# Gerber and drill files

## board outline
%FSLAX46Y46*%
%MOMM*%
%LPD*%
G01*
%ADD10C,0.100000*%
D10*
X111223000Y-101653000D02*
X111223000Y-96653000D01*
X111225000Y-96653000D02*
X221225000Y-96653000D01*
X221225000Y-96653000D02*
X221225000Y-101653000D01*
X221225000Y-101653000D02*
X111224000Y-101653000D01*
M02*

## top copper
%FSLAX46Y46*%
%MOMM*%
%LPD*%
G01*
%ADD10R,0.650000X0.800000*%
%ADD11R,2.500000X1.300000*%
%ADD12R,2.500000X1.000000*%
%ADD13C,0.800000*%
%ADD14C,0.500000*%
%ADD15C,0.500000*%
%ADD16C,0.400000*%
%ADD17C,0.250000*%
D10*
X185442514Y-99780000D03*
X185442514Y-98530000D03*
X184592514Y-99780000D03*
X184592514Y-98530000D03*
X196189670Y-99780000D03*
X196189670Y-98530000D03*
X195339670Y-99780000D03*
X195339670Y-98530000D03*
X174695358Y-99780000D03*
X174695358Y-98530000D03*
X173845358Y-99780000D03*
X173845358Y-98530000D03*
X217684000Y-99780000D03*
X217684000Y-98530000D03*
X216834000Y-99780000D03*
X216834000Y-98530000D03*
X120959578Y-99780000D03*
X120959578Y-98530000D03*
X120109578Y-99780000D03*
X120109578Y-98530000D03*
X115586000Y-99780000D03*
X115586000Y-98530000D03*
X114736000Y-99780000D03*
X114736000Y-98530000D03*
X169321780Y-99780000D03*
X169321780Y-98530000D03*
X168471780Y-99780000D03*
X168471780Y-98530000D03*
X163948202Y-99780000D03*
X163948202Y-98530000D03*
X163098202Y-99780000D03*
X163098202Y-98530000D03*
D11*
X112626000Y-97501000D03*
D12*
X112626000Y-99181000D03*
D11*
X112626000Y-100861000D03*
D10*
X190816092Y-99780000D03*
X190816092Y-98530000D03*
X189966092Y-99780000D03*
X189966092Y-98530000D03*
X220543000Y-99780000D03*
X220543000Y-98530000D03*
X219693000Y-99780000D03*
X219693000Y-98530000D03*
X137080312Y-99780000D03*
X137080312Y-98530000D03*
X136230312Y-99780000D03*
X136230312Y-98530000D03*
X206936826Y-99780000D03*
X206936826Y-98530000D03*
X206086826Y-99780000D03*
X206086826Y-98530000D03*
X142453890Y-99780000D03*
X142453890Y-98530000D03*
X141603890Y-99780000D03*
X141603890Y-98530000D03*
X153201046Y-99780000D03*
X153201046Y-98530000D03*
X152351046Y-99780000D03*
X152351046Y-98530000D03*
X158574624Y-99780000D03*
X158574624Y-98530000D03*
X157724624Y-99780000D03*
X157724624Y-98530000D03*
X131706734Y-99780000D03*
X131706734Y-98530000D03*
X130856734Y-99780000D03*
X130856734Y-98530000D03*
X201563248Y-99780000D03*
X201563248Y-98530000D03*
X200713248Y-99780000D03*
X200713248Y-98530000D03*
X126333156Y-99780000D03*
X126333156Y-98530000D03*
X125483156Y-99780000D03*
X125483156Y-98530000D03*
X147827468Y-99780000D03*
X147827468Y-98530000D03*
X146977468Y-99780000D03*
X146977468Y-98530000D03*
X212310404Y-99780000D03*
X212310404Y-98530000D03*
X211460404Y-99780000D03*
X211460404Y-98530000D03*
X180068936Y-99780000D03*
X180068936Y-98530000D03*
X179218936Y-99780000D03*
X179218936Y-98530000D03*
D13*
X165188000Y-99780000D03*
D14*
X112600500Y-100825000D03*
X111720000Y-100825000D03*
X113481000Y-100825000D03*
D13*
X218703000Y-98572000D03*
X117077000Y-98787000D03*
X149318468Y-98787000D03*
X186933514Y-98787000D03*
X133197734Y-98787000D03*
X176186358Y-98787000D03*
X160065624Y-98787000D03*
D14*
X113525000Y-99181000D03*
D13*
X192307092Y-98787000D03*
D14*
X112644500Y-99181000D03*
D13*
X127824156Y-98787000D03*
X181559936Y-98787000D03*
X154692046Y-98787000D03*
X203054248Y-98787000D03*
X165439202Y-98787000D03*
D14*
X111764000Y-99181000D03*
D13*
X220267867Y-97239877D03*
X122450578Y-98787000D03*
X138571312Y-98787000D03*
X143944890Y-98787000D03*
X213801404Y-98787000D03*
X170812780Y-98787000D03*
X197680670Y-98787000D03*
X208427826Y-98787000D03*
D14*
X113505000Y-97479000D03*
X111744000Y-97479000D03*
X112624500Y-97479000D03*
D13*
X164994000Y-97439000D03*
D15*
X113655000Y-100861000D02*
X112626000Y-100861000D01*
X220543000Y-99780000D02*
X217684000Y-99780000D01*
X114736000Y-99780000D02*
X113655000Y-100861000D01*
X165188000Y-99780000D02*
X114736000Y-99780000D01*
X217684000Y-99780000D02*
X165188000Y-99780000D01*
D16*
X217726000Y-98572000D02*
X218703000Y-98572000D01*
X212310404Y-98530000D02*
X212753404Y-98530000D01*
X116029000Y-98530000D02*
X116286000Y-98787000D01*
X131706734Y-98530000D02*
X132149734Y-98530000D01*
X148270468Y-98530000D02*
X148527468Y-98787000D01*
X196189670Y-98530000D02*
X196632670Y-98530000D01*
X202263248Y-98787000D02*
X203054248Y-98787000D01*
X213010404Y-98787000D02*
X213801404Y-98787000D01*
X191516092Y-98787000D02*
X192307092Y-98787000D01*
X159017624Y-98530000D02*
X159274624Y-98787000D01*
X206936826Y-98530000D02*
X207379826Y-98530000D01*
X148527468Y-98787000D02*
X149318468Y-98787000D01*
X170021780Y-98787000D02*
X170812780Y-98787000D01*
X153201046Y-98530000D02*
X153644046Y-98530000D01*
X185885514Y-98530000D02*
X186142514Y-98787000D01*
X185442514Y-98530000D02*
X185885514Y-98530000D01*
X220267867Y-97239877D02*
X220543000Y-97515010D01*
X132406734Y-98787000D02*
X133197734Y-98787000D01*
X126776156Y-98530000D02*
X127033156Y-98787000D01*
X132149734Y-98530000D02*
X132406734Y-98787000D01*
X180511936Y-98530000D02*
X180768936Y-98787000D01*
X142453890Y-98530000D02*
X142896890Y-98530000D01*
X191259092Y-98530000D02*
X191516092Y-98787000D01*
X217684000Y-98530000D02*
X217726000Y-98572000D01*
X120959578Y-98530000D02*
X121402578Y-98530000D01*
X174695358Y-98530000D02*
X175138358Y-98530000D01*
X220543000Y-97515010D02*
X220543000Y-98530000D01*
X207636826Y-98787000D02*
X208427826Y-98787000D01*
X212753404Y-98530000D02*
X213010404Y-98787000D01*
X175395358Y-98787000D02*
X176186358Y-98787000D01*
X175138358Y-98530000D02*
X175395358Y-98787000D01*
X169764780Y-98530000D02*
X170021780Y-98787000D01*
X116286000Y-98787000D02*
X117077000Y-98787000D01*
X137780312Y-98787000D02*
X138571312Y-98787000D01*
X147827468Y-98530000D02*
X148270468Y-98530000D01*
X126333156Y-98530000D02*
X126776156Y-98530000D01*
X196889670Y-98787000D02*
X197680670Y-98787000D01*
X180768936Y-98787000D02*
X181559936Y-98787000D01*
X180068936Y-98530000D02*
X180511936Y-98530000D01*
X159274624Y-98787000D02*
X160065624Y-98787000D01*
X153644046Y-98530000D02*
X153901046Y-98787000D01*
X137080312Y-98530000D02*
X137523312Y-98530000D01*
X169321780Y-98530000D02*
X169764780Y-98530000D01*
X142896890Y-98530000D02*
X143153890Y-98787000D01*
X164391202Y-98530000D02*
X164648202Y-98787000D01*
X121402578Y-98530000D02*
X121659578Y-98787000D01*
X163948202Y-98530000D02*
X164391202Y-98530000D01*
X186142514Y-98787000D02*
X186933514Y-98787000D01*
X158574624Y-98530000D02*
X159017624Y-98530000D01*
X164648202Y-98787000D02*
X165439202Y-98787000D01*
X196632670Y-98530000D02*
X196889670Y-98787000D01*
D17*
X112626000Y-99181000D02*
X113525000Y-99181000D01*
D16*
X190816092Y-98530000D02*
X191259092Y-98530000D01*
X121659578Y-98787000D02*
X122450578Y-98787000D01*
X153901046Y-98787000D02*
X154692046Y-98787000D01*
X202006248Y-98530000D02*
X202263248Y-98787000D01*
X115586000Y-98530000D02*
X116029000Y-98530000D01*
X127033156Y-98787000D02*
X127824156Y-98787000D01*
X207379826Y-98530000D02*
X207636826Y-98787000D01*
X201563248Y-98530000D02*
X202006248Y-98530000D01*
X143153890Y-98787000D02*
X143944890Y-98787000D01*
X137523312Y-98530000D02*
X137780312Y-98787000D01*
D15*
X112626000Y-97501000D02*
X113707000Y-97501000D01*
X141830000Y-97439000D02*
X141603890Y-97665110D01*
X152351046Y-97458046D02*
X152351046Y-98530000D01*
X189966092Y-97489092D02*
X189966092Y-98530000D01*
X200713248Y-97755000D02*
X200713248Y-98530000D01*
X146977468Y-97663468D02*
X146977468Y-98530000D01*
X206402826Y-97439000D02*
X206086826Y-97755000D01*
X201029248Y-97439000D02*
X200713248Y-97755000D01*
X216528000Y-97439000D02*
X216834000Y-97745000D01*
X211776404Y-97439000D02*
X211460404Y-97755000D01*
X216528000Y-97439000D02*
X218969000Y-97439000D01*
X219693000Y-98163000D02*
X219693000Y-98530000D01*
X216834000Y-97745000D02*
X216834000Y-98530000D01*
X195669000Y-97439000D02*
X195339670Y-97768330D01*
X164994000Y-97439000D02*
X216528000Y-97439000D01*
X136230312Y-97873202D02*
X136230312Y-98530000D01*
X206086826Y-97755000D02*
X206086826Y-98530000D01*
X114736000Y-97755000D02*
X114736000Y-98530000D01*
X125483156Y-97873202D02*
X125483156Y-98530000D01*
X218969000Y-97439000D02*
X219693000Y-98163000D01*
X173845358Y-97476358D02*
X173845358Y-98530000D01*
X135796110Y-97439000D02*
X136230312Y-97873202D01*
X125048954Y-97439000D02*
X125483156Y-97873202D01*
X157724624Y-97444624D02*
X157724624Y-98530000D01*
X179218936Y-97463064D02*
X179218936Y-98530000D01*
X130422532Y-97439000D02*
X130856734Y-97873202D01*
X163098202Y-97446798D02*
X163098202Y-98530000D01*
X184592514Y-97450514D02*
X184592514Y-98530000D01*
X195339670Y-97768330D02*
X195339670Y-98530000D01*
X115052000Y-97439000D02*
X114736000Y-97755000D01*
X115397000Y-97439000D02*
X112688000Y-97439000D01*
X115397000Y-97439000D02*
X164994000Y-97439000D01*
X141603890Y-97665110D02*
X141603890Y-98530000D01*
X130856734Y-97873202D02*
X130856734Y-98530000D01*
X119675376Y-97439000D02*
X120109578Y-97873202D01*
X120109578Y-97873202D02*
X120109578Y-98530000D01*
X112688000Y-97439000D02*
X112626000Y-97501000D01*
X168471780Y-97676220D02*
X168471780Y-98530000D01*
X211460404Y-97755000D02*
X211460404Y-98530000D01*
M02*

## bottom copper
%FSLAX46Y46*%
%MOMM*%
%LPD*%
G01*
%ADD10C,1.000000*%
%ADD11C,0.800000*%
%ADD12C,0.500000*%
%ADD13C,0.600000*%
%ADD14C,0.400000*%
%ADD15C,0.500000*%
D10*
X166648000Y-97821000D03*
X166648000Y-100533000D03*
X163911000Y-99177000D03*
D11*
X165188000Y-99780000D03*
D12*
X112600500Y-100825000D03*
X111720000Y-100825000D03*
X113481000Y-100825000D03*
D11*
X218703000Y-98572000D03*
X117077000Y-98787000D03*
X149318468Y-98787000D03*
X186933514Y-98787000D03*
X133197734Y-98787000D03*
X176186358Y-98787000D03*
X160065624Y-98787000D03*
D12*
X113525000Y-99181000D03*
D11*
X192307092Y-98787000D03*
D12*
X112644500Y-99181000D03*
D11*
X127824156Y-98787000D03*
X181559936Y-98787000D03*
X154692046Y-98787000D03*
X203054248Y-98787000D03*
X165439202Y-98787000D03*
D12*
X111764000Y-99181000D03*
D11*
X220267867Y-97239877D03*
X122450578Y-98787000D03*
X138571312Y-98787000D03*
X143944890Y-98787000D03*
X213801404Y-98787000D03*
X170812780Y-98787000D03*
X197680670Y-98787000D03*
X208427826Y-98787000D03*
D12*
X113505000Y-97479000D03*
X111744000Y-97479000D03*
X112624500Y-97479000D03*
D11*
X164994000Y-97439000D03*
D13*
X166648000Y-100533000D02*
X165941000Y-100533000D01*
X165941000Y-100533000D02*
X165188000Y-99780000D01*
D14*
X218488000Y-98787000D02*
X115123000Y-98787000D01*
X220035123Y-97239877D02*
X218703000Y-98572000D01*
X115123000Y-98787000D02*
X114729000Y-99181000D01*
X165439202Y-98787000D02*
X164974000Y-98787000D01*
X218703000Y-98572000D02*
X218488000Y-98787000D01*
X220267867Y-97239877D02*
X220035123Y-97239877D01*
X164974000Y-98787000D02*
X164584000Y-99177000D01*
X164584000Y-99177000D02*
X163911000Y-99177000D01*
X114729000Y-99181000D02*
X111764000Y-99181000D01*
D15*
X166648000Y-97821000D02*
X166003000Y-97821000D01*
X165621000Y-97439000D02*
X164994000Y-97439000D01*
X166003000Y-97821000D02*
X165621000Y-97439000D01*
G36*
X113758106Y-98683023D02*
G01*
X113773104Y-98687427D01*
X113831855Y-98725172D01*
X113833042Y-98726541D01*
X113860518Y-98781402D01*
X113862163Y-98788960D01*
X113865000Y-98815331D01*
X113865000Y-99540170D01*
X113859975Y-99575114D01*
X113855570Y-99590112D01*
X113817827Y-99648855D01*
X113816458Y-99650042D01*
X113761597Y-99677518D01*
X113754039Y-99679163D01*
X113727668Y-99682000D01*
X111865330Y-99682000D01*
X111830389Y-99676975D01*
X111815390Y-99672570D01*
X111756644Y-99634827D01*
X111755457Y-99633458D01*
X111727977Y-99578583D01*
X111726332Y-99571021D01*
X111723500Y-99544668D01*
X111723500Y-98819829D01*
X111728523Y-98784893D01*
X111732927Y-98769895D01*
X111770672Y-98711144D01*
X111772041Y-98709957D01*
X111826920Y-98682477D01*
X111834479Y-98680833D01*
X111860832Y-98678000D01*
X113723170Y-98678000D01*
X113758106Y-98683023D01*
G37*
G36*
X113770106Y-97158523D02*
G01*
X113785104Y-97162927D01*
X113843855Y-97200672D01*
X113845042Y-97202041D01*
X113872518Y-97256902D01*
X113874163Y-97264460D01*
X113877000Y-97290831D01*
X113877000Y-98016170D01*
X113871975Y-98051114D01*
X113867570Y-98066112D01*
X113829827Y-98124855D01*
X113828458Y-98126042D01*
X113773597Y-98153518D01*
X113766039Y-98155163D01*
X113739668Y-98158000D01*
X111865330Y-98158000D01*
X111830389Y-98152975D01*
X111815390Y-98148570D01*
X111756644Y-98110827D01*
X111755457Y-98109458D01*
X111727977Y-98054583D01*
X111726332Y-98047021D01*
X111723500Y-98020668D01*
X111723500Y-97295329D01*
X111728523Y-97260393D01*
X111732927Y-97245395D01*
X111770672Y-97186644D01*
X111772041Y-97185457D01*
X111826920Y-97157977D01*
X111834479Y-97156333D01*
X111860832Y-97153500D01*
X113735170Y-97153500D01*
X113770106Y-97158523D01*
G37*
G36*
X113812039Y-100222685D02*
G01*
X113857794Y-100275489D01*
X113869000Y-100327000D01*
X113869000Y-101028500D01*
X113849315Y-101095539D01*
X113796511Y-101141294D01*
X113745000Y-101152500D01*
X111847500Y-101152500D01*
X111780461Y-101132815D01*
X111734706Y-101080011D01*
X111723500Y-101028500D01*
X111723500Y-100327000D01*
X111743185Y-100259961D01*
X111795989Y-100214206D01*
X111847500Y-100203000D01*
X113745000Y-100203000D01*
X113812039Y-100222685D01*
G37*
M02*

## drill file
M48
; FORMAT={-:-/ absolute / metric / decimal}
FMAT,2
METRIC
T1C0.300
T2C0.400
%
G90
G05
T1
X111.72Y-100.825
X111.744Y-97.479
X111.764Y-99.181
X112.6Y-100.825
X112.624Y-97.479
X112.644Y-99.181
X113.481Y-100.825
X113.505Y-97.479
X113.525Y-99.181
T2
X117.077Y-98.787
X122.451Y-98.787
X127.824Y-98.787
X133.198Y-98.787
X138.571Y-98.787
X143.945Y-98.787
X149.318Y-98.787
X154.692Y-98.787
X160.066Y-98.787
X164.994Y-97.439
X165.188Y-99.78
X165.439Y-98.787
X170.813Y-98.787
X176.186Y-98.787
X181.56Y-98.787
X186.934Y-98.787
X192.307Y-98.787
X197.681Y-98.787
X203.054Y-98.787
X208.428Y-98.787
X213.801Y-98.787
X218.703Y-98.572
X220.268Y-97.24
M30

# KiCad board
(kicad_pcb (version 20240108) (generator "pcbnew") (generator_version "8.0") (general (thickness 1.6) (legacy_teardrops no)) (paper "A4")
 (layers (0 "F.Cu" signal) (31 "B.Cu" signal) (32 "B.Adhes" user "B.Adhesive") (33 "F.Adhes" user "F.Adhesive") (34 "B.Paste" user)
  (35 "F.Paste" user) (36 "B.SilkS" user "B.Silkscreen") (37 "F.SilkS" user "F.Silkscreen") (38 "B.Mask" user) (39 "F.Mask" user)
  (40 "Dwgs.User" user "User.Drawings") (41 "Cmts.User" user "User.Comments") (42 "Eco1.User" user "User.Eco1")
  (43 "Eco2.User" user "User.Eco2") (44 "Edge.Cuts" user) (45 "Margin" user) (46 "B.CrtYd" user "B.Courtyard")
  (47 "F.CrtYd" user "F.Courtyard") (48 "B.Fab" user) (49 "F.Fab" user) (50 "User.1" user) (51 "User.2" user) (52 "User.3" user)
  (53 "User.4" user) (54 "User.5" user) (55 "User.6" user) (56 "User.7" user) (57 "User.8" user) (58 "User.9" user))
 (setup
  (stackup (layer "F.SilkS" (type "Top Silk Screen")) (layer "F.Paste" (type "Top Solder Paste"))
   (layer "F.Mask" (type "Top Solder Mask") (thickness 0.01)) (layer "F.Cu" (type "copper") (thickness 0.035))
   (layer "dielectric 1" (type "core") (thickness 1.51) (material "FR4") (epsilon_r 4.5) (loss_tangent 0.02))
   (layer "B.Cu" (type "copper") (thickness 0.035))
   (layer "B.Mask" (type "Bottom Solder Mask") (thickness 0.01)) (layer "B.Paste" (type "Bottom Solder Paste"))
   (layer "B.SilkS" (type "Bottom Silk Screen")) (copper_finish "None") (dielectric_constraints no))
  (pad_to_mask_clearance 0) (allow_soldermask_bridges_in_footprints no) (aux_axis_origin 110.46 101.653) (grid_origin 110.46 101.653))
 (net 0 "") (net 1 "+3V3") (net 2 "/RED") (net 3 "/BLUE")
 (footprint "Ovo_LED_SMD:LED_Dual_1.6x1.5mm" (layer "F.Cu") (at 185.017514 99.155 90)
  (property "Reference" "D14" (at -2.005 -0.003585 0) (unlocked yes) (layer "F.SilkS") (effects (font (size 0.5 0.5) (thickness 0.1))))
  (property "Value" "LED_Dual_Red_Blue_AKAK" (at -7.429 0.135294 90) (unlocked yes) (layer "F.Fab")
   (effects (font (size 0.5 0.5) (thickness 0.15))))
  (pad "1" smd rect (at -0.625 0.425 90) (size 0.8 0.65) (layers "F.Cu" "F.Paste" "F.Mask") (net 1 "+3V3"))
  (pad "2" smd rect (at 0.625 0.425 90) (size 0.8 0.65) (layers "F.Cu" "F.Paste" "F.Mask") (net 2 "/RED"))
  (pad "3" smd rect (at -0.625 -0.425 90) (size 0.8 0.65) (layers "F.Cu" "F.Paste" "F.Mask") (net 1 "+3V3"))
  (pad "4" smd rect (at 0.625 -0.425 90) (size 0.8 0.65) (layers "F.Cu" "F.Paste" "F.Mask") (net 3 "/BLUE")))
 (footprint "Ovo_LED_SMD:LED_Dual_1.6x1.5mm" (layer "F.Cu") (at 195.76467 99.155 90)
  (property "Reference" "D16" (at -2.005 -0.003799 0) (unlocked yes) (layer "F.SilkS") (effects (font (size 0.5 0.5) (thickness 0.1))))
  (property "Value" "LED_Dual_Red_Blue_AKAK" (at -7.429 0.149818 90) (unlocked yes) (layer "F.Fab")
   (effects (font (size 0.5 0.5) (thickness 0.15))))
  (pad "1" smd rect (at -0.625 0.425 90) (size 0.8 0.65) (layers "F.Cu" "F.Paste" "F.Mask") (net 1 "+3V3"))
  (pad "2" smd rect (at 0.625 0.425 90) (size 0.8 0.65) (layers "F.Cu" "F.Paste" "F.Mask") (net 2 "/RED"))
  (pad "3" smd rect (at -0.625 -0.425 90) (size 0.8 0.65) (layers "F.Cu" "F.Paste" "F.Mask") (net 1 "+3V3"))
  (pad "4" smd rect (at 0.625 -0.425 90) (size 0.8 0.65) (layers "F.Cu" "F.Paste" "F.Mask") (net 3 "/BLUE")))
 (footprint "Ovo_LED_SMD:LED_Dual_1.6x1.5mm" (layer "F.Cu") (at 174.270358 99.155 90)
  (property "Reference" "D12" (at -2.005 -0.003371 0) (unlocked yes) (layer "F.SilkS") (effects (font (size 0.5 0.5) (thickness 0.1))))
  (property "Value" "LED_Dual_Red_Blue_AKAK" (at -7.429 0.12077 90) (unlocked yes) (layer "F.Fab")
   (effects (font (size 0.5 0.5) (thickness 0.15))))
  (pad "1" smd rect (at -0.625 0.425 90) (size 0.8 0.65) (layers "F.Cu" "F.Paste" "F.Mask") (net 1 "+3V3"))
  (pad "2" smd rect (at 0.625 0.425 90) (size 0.8 0.65) (layers "F.Cu" "F.Paste" "F.Mask") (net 2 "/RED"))
  (pad "3" smd rect (at -0.625 -0.425 90) (size 0.8 0.65) (layers "F.Cu" "F.Paste" "F.Mask") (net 1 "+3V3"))
  (pad "4" smd rect (at 0.625 -0.425 90) (size 0.8 0.65) (layers "F.Cu" "F.Paste" "F.Mask") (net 3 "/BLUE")))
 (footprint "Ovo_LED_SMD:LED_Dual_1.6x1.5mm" (layer "F.Cu") (at 217.259 99.155 90)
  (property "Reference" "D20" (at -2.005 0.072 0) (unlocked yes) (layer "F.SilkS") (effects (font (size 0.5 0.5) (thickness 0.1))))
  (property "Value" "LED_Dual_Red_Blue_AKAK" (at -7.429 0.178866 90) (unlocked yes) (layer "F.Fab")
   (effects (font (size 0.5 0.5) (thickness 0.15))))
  (pad "1" smd rect (at -0.625 0.425 90) (size 0.8 0.65) (layers "F.Cu" "F.Paste" "F.Mask") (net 1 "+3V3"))
  (pad "2" smd rect (at 0.625 0.425 90) (size 0.8 0.65) (layers "F.Cu" "F.Paste" "F.Mask") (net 2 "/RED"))
  (pad "3" smd rect (at -0.625 -0.425 90) (size 0.8 0.65) (layers "F.Cu" "F.Paste" "F.Mask") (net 1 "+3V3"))
  (pad "4" smd rect (at 0.625 -0.425 90) (size 0.8 0.65) (layers "F.Cu" "F.Paste" "F.Mask") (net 3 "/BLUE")))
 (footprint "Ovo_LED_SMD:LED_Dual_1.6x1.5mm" (layer "F.Cu") (at 120.534578 99.155 90)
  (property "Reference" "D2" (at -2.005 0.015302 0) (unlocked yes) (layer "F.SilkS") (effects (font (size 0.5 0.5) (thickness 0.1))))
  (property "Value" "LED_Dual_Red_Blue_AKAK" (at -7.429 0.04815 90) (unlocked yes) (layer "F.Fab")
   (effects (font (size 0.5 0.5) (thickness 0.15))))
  (pad "1" smd rect (at -0.625 0.425 90) (size 0.8 0.65) (layers "F.Cu" "F.Paste" "F.Mask") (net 1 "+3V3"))
  (pad "2" smd rect (at 0.625 0.425 90) (size 0.8 0.65) (layers "F.Cu" "F.Paste" "F.Mask") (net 2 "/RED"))
  (pad "3" smd rect (at -0.625 -0.425 90) (size 0.8 0.65) (layers "F.Cu" "F.Paste" "F.Mask") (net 1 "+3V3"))
  (pad "4" smd rect (at 0.625 -0.425 90) (size 0.8 0.65) (layers "F.Cu" "F.Paste" "F.Mask") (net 3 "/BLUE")))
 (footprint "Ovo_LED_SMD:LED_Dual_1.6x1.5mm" (layer "F.Cu") (at 115.161 99.155 90)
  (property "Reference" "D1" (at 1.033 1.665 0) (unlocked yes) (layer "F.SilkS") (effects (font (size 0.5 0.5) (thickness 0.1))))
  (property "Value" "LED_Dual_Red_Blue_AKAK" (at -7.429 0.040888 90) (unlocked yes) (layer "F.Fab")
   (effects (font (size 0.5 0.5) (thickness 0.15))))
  (pad "1" smd rect (at -0.625 0.425 90) (size 0.8 0.65) (layers "F.Cu" "F.Paste" "F.Mask") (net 1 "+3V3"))
  (pad "2" smd rect (at 0.625 0.425 90) (size 0.8 0.65) (layers "F.Cu" "F.Paste" "F.Mask") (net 2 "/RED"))
  (pad "3" smd rect (at -0.625 -0.425 90) (size 0.8 0.65) (layers "F.Cu" "F.Paste" "F.Mask") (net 1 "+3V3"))
  (pad "4" smd rect (at 0.625 -0.425 90) (size 0.8 0.65) (layers "F.Cu" "F.Paste" "F.Mask") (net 3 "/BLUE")))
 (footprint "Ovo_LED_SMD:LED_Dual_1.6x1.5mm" (layer "F.Cu") (at 168.89678 99.155 90)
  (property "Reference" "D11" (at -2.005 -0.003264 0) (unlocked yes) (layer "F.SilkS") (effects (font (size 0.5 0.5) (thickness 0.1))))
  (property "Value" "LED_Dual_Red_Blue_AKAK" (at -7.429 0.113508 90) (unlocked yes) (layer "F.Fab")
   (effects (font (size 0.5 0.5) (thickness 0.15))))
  (pad "1" smd rect (at -0.625 0.425 90) (size 0.8 0.65) (layers "F.Cu" "F.Paste" "F.Mask") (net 1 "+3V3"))
  (pad "2" smd rect (at 0.625 0.425 90) (size 0.8 0.65) (layers "F.Cu" "F.Paste" "F.Mask") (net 2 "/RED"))
  (pad "3" smd rect (at -0.625 -0.425 90) (size 0.8 0.65) (layers "F.Cu" "F.Paste" "F.Mask") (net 1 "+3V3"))
  (pad "4" smd rect (at 0.625 -0.425 90) (size 0.8 0.65) (layers "F.Cu" "F.Paste" "F.Mask") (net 3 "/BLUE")))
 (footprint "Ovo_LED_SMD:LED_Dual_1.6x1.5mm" (layer "F.Cu") (at 163.523202 99.155 90)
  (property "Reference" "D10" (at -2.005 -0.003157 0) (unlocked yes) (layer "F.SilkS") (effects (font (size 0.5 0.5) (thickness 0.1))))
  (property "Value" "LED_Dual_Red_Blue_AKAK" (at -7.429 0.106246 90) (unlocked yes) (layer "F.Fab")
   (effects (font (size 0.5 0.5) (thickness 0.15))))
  (pad "1" smd rect (at -0.625 0.425 90) (size 0.8 0.65) (layers "F.Cu" "F.Paste" "F.Mask") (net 1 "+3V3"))
  (pad "2" smd rect (at 0.625 0.425 90) (size 0.8 0.65) (layers "F.Cu" "F.Paste" "F.Mask") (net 2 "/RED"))
  (pad "3" smd rect (at -0.625 -0.425 90) (size 0.8 0.65) (layers "F.Cu" "F.Paste" "F.Mask") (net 1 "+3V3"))
  (pad "4" smd rect (at 0.625 -0.425 90) (size 0.8 0.65) (layers "F.Cu" "F.Paste" "F.Mask") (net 3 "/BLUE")))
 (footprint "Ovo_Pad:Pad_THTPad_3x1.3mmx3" (layer "F.Cu") (at 112.666 97.511)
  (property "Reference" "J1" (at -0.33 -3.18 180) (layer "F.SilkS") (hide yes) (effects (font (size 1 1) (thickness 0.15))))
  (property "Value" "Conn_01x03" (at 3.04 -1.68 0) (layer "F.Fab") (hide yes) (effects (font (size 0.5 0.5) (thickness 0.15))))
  (pad "1" smd rect (at -0.04 -0.01 180) (size 2.5 1.3) (layers "F.Cu" "F.Paste" "F.Mask") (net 3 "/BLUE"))
  (pad "2" smd rect (at -0.04 1.67 180) (size 2.5 1) (layers "F.Cu" "F.Paste" "F.Mask") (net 2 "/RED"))
  (pad "3" smd rect (at -0.04 3.35 180) (size 2.5 1.3) (layers "F.Cu" "F.Paste" "F.Mask") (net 1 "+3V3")))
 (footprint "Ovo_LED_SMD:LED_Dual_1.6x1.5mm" (layer "F.Cu") (at 190.391092 99.155 90)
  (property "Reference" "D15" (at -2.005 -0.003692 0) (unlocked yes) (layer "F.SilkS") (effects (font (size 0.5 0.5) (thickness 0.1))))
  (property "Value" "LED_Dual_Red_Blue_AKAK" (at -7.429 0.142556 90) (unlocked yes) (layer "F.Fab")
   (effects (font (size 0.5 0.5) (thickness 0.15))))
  (pad "1" smd rect (at -0.625 0.425 90) (size 0.8 0.65) (layers "F.Cu" "F.Paste" "F.Mask") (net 1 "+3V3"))
  (pad "2" smd rect (at 0.625 0.425 90) (size 0.8 0.65) (layers "F.Cu" "F.Paste" "F.Mask") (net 2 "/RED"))
  (pad "3" smd rect (at -0.625 -0.425 90) (size 0.8 0.65) (layers "F.Cu" "F.Paste" "F.Mask") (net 1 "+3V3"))
  (pad "4" smd rect (at 0.625 -0.425 90) (size 0.8 0.65) (layers "F.Cu" "F.Paste" "F.Mask") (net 3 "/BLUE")))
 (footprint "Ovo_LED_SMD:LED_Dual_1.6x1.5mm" (layer "F.Cu") (at 220.118 99.155 90)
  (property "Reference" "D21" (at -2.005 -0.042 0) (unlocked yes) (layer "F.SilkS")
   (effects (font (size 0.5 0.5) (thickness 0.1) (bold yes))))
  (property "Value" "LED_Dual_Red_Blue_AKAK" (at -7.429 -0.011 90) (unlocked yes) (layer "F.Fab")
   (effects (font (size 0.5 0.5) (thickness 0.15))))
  (pad "1" smd rect (at -0.625 0.425 90) (size 0.8 0.65) (layers "F.Cu" "F.Paste" "F.Mask") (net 1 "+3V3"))
  (pad "2" smd rect (at 0.625 0.425 90) (size 0.8 0.65) (layers "F.Cu" "F.Paste" "F.Mask") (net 2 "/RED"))
  (pad "3" smd rect (at -0.625 -0.425 90) (size 0.8 0.65) (layers "F.Cu" "F.Paste" "F.Mask") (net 1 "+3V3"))
  (pad "4" smd rect (at 0.625 -0.425 90) (size 0.8 0.65) (layers "F.Cu" "F.Paste" "F.Mask") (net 3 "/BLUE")))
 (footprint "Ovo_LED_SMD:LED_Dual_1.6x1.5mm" (layer "F.Cu") (at 136.655312 99.155 90)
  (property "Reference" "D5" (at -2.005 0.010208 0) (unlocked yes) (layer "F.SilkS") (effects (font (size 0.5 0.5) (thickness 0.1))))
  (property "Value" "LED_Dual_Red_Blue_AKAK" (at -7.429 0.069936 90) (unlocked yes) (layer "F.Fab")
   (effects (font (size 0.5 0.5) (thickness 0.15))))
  (pad "1" smd rect (at -0.625 0.425 90) (size 0.8 0.65) (layers "F.Cu" "F.Paste" "F.Mask") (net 1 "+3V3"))
  (pad "2" smd rect (at 0.625 0.425 90) (size 0.8 0.65) (layers "F.Cu" "F.Paste" "F.Mask") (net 2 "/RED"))
  (pad "3" smd rect (at -0.625 -0.425 90) (size 0.8 0.65) (layers "F.Cu" "F.Paste" "F.Mask") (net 1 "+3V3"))
  (pad "4" smd rect (at 0.625 -0.425 90) (size 0.8 0.65) (layers "F.Cu" "F.Paste" "F.Mask") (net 3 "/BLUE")))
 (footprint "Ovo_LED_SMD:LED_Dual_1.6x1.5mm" (layer "F.Cu") (at 206.511826 99.155 90)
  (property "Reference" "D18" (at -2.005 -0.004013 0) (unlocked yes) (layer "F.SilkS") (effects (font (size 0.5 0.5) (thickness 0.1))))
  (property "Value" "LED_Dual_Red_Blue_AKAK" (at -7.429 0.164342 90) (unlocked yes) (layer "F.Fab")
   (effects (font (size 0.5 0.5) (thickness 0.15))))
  (pad "1" smd rect (at -0.625 0.425 90) (size 0.8 0.65) (layers "F.Cu" "F.Paste" "F.Mask") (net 1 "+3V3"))
  (pad "2" smd rect (at 0.625 0.425 90) (size 0.8 0.65) (layers "F.Cu" "F.Paste" "F.Mask") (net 2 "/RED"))
  (pad "3" smd rect (at -0.625 -0.425 90) (size 0.8 0.65) (layers "F.Cu" "F.Paste" "F.Mask") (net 1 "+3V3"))
  (pad "4" smd rect (at 0.625 -0.425 90) (size 0.8 0.65) (layers "F.Cu" "F.Paste" "F.Mask") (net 3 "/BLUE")))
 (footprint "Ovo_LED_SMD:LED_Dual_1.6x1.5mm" (layer "F.Cu") (at 142.02889 99.155 90)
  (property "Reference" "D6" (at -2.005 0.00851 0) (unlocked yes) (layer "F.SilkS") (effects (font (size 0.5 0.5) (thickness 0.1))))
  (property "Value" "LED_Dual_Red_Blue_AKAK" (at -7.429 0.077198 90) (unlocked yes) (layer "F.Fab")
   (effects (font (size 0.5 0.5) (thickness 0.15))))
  (pad "1" smd rect (at -0.625 0.425 90) (size 0.8 0.65) (layers "F.Cu" "F.Paste" "F.Mask") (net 1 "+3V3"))
  (pad "2" smd rect (at 0.625 0.425 90) (size 0.8 0.65) (layers "F.Cu" "F.Paste" "F.Mask") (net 2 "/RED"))
  (pad "3" smd rect (at -0.625 -0.425 90) (size 0.8 0.65) (layers "F.Cu" "F.Paste" "F.Mask") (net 1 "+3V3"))
  (pad "4" smd rect (at 0.625 -0.425 90) (size 0.8 0.65) (layers "F.Cu" "F.Paste" "F.Mask") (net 3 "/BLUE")))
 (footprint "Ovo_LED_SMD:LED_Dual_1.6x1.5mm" (layer "F.Cu") (at 152.776046 99.155 90)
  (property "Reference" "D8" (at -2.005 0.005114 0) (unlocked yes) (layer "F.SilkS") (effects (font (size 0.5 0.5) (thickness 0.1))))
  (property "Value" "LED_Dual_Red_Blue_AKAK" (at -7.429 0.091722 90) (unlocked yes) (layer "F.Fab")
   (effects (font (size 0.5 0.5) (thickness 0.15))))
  (pad "1" smd rect (at -0.625 0.425 90) (size 0.8 0.65) (layers "F.Cu" "F.Paste" "F.Mask") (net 1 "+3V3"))
  (pad "2" smd rect (at 0.625 0.425 90) (size 0.8 0.65) (layers "F.Cu" "F.Paste" "F.Mask") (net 2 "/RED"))
  (pad "3" smd rect (at -0.625 -0.425 90) (size 0.8 0.65) (layers "F.Cu" "F.Paste" "F.Mask") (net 1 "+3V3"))
  (pad "4" smd rect (at 0.625 -0.425 90) (size 0.8 0.65) (layers "F.Cu" "F.Paste" "F.Mask") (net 3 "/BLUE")))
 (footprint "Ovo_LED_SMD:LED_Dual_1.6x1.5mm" (layer "F.Cu") (at 158.149624 99.155 90)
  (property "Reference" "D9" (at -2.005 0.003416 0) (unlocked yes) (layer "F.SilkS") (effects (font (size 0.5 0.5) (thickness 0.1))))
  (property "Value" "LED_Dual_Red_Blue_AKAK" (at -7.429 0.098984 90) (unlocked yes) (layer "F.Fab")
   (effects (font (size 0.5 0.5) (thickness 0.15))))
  (pad "1" smd rect (at -0.625 0.425 90) (size 0.8 0.65) (layers "F.Cu" "F.Paste" "F.Mask") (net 1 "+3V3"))
  (pad "2" smd rect (at 0.625 0.425 90) (size 0.8 0.65) (layers "F.Cu" "F.Paste" "F.Mask") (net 2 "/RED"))
  (pad "3" smd rect (at -0.625 -0.425 90) (size 0.8 0.65) (layers "F.Cu" "F.Paste" "F.Mask") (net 1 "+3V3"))
  (pad "4" smd rect (at 0.625 -0.425 90) (size 0.8 0.65) (layers "F.Cu" "F.Paste" "F.Mask") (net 3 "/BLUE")))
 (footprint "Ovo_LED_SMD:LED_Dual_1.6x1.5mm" (layer "F.Cu") (at 131.281734 99.155 90)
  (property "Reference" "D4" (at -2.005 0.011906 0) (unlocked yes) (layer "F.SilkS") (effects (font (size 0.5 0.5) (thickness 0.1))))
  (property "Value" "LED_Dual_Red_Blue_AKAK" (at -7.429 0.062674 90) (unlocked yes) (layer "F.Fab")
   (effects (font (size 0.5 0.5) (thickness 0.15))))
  (pad "1" smd rect (at -0.625 0.425 90) (size 0.8 0.65) (layers "F.Cu" "F.Paste" "F.Mask") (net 1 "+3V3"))
  (pad "2" smd rect (at 0.625 0.425 90) (size 0.8 0.65) (layers "F.Cu" "F.Paste" "F.Mask") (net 2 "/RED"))
  (pad "3" smd rect (at -0.625 -0.425 90) (size 0.8 0.65) (layers "F.Cu" "F.Paste" "F.Mask") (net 1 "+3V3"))
  (pad "4" smd rect (at 0.625 -0.425 90) (size 0.8 0.65) (layers "F.Cu" "F.Paste" "F.Mask") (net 3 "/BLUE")))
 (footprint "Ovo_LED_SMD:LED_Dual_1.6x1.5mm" (layer "F.Cu") (at 201.138248 99.155 90)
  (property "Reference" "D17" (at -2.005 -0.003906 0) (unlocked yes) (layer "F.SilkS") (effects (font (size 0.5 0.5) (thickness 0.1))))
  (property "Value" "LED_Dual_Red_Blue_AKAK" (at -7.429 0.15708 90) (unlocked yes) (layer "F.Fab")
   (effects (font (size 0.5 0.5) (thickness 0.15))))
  (pad "1" smd rect (at -0.625 0.425 90) (size 0.8 0.65) (layers "F.Cu" "F.Paste" "F.Mask") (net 1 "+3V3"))
  (pad "2" smd rect (at 0.625 0.425 90) (size 0.8 0.65) (layers "F.Cu" "F.Paste" "F.Mask") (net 2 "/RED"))
  (pad "3" smd rect (at -0.625 -0.425 90) (size 0.8 0.65) (layers "F.Cu" "F.Paste" "F.Mask") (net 1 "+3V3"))
  (pad "4" smd rect (at 0.625 -0.425 90) (size 0.8 0.65) (layers "F.Cu" "F.Paste" "F.Mask") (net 3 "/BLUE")))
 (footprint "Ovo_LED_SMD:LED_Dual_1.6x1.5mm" (layer "F.Cu") (at 125.908156 99.155 90)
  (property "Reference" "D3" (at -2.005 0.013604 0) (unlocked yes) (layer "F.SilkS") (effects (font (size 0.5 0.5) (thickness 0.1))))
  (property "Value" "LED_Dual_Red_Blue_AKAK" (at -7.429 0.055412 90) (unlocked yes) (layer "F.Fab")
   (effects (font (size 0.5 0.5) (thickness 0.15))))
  (pad "1" smd rect (at -0.625 0.425 90) (size 0.8 0.65) (layers "F.Cu" "F.Paste" "F.Mask") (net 1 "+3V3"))
  (pad "2" smd rect (at 0.625 0.425 90) (size 0.8 0.65) (layers "F.Cu" "F.Paste" "F.Mask") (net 2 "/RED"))
  (pad "3" smd rect (at -0.625 -0.425 90) (size 0.8 0.65) (layers "F.Cu" "F.Paste" "F.Mask") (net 1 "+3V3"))
  (pad "4" smd rect (at 0.625 -0.425 90) (size 0.8 0.65) (layers "F.Cu" "F.Paste" "F.Mask") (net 3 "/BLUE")))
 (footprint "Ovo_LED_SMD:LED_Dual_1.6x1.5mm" (layer "F.Cu") (at 147.402468 99.155 90)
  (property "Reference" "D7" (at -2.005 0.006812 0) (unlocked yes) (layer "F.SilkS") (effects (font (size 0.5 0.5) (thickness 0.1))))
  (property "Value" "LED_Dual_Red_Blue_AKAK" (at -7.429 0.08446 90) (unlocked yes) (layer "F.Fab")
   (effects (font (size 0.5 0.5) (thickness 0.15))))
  (pad "1" smd rect (at -0.625 0.425 90) (size 0.8 0.65) (layers "F.Cu" "F.Paste" "F.Mask") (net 1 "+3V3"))
  (pad "2" smd rect (at 0.625 0.425 90) (size 0.8 0.65) (layers "F.Cu" "F.Paste" "F.Mask") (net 2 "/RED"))
  (pad "3" smd rect (at -0.625 -0.425 90) (size 0.8 0.65) (layers "F.Cu" "F.Paste" "F.Mask") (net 1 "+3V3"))
  (pad "4" smd rect (at 0.625 -0.425 90) (size 0.8 0.65) (layers "F.Cu" "F.Paste" "F.Mask") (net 3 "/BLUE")))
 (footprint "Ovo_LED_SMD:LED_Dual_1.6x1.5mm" (layer "F.Cu") (at 211.885404 99.155 90)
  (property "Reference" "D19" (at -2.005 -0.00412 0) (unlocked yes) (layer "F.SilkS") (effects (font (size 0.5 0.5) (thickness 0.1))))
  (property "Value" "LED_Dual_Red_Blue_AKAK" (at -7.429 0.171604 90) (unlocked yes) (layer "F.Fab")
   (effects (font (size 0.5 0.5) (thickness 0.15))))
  (pad "1" smd rect (at -0.625 0.425 90) (size 0.8 0.65) (layers "F.Cu" "F.Paste" "F.Mask") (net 1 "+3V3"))
  (pad "2" smd rect (at 0.625 0.425 90) (size 0.8 0.65) (layers "F.Cu" "F.Paste" "F.Mask") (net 2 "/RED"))
  (pad "3" smd rect (at -0.625 -0.425 90) (size 0.8 0.65) (layers "F.Cu" "F.Paste" "F.Mask") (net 1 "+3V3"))
  (pad "4" smd rect (at 0.625 -0.425 90) (size 0.8 0.65) (layers "F.Cu" "F.Paste" "F.Mask") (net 3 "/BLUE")))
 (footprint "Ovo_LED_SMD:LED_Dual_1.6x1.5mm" (layer "F.Cu") (at 179.643936 99.155 90)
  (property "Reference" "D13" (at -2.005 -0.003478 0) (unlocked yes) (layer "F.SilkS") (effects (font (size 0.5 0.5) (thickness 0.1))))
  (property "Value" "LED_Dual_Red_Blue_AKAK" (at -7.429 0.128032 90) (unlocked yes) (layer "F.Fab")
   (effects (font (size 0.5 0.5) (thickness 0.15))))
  (pad "1" smd rect (at -0.625 0.425 90) (size 0.8 0.65) (layers "F.Cu" "F.Paste" "F.Mask") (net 1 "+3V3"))
  (pad "2" smd rect (at 0.625 0.425 90) (size 0.8 0.65) (layers "F.Cu" "F.Paste" "F.Mask") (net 2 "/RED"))
  (pad "3" smd rect (at -0.625 -0.425 90) (size 0.8 0.65) (layers "F.Cu" "F.Paste" "F.Mask") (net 1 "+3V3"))
  (pad "4" smd rect (at 0.625 -0.425 90) (size 0.8 0.65) (layers "F.Cu" "F.Paste" "F.Mask") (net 3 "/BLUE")))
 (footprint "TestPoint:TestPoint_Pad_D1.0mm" (layer "B.Cu") (at 166.648 97.821 180)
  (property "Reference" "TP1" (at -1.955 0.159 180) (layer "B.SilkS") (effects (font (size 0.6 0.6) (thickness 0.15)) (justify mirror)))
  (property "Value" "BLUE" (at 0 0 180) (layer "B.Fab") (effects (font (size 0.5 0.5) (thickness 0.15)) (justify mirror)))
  (pad "1" smd circle (at 0 0 180) (size 1 1) (layers "B.Cu" "B.Mask") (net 3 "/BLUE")))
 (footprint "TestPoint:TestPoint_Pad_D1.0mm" (layer "B.Cu") (at 166.648 100.533 180)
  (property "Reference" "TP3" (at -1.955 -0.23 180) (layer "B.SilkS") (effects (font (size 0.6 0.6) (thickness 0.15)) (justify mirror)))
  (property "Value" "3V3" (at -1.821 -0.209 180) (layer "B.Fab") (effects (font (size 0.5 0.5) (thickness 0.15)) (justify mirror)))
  (pad "1" smd circle (at 0 0 180) (size 1 1) (layers "B.Cu" "B.Mask") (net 1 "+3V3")))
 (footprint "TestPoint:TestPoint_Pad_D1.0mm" (layer "B.Cu") (at 163.911 99.177 180)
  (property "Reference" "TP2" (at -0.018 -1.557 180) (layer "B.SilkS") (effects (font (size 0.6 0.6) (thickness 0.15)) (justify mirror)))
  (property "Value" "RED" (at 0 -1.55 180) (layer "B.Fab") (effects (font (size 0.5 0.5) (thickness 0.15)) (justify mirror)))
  (pad "1" smd circle (at 0 0 180) (size 1 1) (layers "B.Cu" "B.Mask") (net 2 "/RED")))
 (gr_line (start 111.223 101.653) (end 111.223 96.653) (stroke (width 0.1) (type default)) (layer "Edge.Cuts"))
 (gr_line (start 111.225 96.653) (end 221.225 96.653) (stroke (width 0.1) (type default)) (layer "Edge.Cuts"))
 (gr_line (start 221.225 96.653) (end 221.225 101.653) (stroke (width 0.1) (type default)) (layer "Edge.Cuts"))
 (gr_line (start 221.225 101.653) (end 111.224 101.653) (stroke (width 0.1) (type default)) (layer "Edge.Cuts"))
 (segment (start 113.655 100.861) (end 112.626 100.861) (width 0.5) (layer "F.Cu") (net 1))
 (segment (start 220.543 99.78) (end 217.684 99.78) (width 0.5) (layer "F.Cu") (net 1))
 (segment (start 114.736 99.78) (end 113.655 100.861) (width 0.5) (layer "F.Cu") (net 1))
 (segment (start 165.188 99.78) (end 114.736 99.78) (width 0.5) (layer "F.Cu") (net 1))
 (segment (start 217.684 99.78) (end 165.188 99.78) (width 0.5) (layer "F.Cu") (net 1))
 (via (at 165.188 99.78) (size 0.8) (drill 0.4) (layers "F.Cu" "B.Cu") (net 1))
 (via (at 112.6005 100.825) (size 0.5) (drill 0.3) (layers "F.Cu" "B.Cu") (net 1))
 (via (at 111.72 100.825) (size 0.5) (drill 0.3) (layers "F.Cu" "B.Cu") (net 1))
 (via (at 113.481 100.825) (size 0.5) (drill 0.3) (layers "F.Cu" "B.Cu") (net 1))
 (segment (start 166.648 100.533) (end 165.941 100.533) (width 0.6) (layer "B.Cu") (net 1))
 (segment (start 165.941 100.533) (end 165.188 99.78) (width 0.6) (layer "B.Cu") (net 1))
 (segment (start 217.726 98.572) (end 218.703 98.572) (width 0.4) (layer "F.Cu") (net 2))
 (segment (start 212.310404 98.53) (end 212.753404 98.53) (width 0.4) (layer "F.Cu") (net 2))
 (segment (start 116.029 98.53) (end 116.286 98.787) (width 0.4) (layer "F.Cu") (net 2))
 (segment (start 131.706734 98.53) (end 132.149734 98.53) (width 0.4) (layer "F.Cu") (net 2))
 (segment (start 148.270468 98.53) (end 148.527468 98.787) (width 0.4) (layer "F.Cu") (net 2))
 (segment (start 196.18967 98.53) (end 196.63267 98.53) (width 0.4) (layer "F.Cu") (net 2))
 (segment (start 202.263248 98.787) (end 203.054248 98.787) (width 0.4) (layer "F.Cu") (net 2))
 (segment (start 213.010404 98.787) (end 213.801404 98.787) (width 0.4) (layer "F.Cu") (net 2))
 (segment (start 191.516092 98.787) (end 192.307092 98.787) (width 0.4) (layer "F.Cu") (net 2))
 (segment (start 159.017624 98.53) (end 159.274624 98.787) (width 0.4) (layer "F.Cu") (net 2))
 (segment (start 206.936826 98.53) (end 207.379826 98.53) (width 0.4) (layer "F.Cu") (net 2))
 (segment (start 148.527468 98.787) (end 149.318468 98.787) (width 0.4) (layer "F.Cu") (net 2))
 (segment (start 170.02178 98.787) (end 170.81278 98.787) (width 0.4) (layer "F.Cu") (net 2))
 (segment (start 153.201046 98.53) (end 153.644046 98.53) (width 0.4) (layer "F.Cu") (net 2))
 (segment (start 185.885514 98.53) (end 186.142514 98.787) (width 0.4) (layer "F.Cu") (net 2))
 (segment (start 185.442514 98.53) (end 185.885514 98.53) (width 0.4) (layer "F.Cu") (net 2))
 (segment (start 220.267867 97.239877) (end 220.543 97.51501) (width 0.4) (layer "F.Cu") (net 2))
 (segment (start 132.406734 98.787) (end 133.197734 98.787) (width 0.4) (layer "F.Cu") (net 2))
 (segment (start 126.776156 98.53) (end 127.033156 98.787) (width 0.4) (layer "F.Cu") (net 2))
 (segment (start 132.149734 98.53) (end 132.406734 98.787) (width 0.4) (layer "F.Cu") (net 2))
 (segment (start 180.511936 98.53) (end 180.768936 98.787) (width 0.4) (layer "F.Cu") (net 2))
 (segment (start 142.45389 98.53) (end 142.89689 98.53) (width 0.4) (layer "F.Cu") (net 2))
 (segment (start 191.259092 98.53) (end 191.516092 98.787) (width 0.4) (layer "F.Cu") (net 2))
 (segment (start 217.684 98.53) (end 217.726 98.572) (width 0.4) (layer "F.Cu") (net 2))
 (segment (start 120.959578 98.53) (end 121.402578 98.53) (width 0.4) (layer "F.Cu") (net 2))
 (segment (start 174.695358 98.53) (end 175.138358 98.53) (width 0.4) (layer "F.Cu") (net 2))
 (segment (start 220.543 97.51501) (end 220.543 98.53) (width 0.4) (layer "F.Cu") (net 2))
 (segment (start 207.636826 98.787) (end 208.427826 98.787) (width 0.4) (layer "F.Cu") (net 2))
 (segment (start 212.753404 98.53) (end 213.010404 98.787) (width 0.4) (layer "F.Cu") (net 2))
 (segment (start 175.395358 98.787) (end 176.186358 98.787) (width 0.4) (layer "F.Cu") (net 2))
 (segment (start 175.138358 98.53) (end 175.395358 98.787) (width 0.4) (layer "F.Cu") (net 2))
 (segment (start 169.76478 98.53) (end 170.02178 98.787) (width 0.4) (layer "F.Cu") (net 2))
 (segment (start 116.286 98.787) (end 117.077 98.787) (width 0.4) (layer "F.Cu") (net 2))
 (segment (start 137.780312 98.787) (end 138.571312 98.787) (width 0.4) (layer "F.Cu") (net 2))
 (segment (start 147.827468 98.53) (end 148.270468 98.53) (width 0.4) (layer "F.Cu") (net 2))
 (segment (start 126.333156 98.53) (end 126.776156 98.53) (width 0.4) (layer "F.Cu") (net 2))
 (segment (start 196.88967 98.787) (end 197.68067 98.787) (width 0.4) (layer "F.Cu") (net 2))
 (segment (start 180.768936 98.787) (end 181.559936 98.787) (width 0.4) (layer "F.Cu") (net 2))
 (segment (start 180.068936 98.53) (end 180.511936 98.53) (width 0.4) (layer "F.Cu") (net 2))
 (segment (start 159.274624 98.787) (end 160.065624 98.787) (width 0.4) (layer "F.Cu") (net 2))
 (segment (start 153.644046 98.53) (end 153.901046 98.787) (width 0.4) (layer "F.Cu") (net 2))
 (segment (start 137.080312 98.53) (end 137.523312 98.53) (width 0.4) (layer "F.Cu") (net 2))
 (segment (start 169.32178 98.53) (end 169.76478 98.53) (width 0.4) (layer "F.Cu") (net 2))
 (segment (start 142.89689 98.53) (end 143.15389 98.787) (width 0.4) (layer "F.Cu") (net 2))
 (segment (start 164.391202 98.53) (end 164.648202 98.787) (width 0.4) (layer "F.Cu") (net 2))
 (segment (start 121.402578 98.53) (end 121.659578 98.787) (width 0.4) (layer "F.Cu") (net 2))
 (segment (start 163.948202 98.53) (end 164.391202 98.53) (width 0.4) (layer "F.Cu") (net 2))
 (segment (start 186.142514 98.787) (end 186.933514 98.787) (width 0.4) (layer "F.Cu") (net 2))
 (segment (start 158.574624 98.53) (end 159.017624 98.53) (width 0.4) (layer "F.Cu") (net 2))
 (segment (start 164.648202 98.787) (end 165.439202 98.787) (width 0.4) (layer "F.Cu") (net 2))
 (segment (start 196.63267 98.53) (end 196.88967 98.787) (width 0.4) (layer "F.Cu") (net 2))
 (segment (start 112.626 99.181) (end 113.525 99.181) (width 0.25) (layer "F.Cu") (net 2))
 (segment (start 190.816092 98.53) (end 191.259092 98.53) (width 0.4) (layer "F.Cu") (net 2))
 (segment (start 121.659578 98.787) (end 122.450578 98.787) (width 0.4) (layer "F.Cu") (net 2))
 (segment (start 153.901046 98.787) (end 154.692046 98.787) (width 0.4) (layer "F.Cu") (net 2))
 (segment (start 202.006248 98.53) (end 202.263248 98.787) (width 0.4) (layer "F.Cu") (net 2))
 (segment (start 115.586 98.53) (end 116.029 98.53) (width 0.4) (layer "F.Cu") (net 2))
 (segment (start 127.033156 98.787) (end 127.824156 98.787) (width 0.4) (layer "F.Cu") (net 2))
 (segment (start 207.379826 98.53) (end 207.636826 98.787) (width 0.4) (layer "F.Cu") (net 2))
 (segment (start 201.563248 98.53) (end 202.006248 98.53) (width 0.4) (layer "F.Cu") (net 2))
 (segment (start 143.15389 98.787) (end 143.94489 98.787) (width 0.4) (layer "F.Cu") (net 2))
 (segment (start 137.523312 98.53) (end 137.780312 98.787) (width 0.4) (layer "F.Cu") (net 2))
 (via (at 218.703 98.572) (size 0.8) (drill 0.4) (layers "F.Cu" "B.Cu") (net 2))
 (via (at 117.077 98.787) (size 0.8) (drill 0.4) (layers "F.Cu" "B.Cu") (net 2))
 (via (at 149.318468 98.787) (size 0.8) (drill 0.4) (layers "F.Cu" "B.Cu") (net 2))
 (via (at 186.933514 98.787) (size 0.8) (drill 0.4) (layers "F.Cu" "B.Cu") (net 2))
 (via (at 133.197734 98.787) (size 0.8) (drill 0.4) (layers "F.Cu" "B.Cu") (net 2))
 (via (at 176.186358 98.787) (size 0.8) (drill 0.4) (layers "F.Cu" "B.Cu") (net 2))
 (via (at 160.065624 98.787) (size 0.8) (drill 0.4) (layers "F.Cu" "B.Cu") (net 2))
 (via (at 113.525 99.181) (size 0.5) (drill 0.3) (layers "F.Cu" "B.Cu") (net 2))
 (via (at 192.307092 98.787) (size 0.8) (drill 0.4) (layers "F.Cu" "B.Cu") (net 2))
 (via (at 112.6445 99.181) (size 0.5) (drill 0.3) (layers "F.Cu" "B.Cu") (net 2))
 (via (at 127.824156 98.787) (size 0.8) (drill 0.4) (layers "F.Cu" "B.Cu") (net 2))
 (via (at 181.559936 98.787) (size 0.8) (drill 0.4) (layers "F.Cu" "B.Cu") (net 2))
 (via (at 154.692046 98.787) (size 0.8) (drill 0.4) (layers "F.Cu" "B.Cu") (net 2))
 (via (at 203.054248 98.787) (size 0.8) (drill 0.4) (layers "F.Cu" "B.Cu") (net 2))
 (via (at 165.439202 98.787) (size 0.8) (drill 0.4) (layers "F.Cu" "B.Cu") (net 2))
 (via (at 111.764 99.181) (size 0.5) (drill 0.3) (layers "F.Cu" "B.Cu") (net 2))
 (via (at 220.267867 97.239877) (size 0.8) (drill 0.4) (layers "F.Cu" "B.Cu") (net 2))
 (via (at 122.450578 98.787) (size 0.8) (drill 0.4) (layers "F.Cu" "B.Cu") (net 2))
 (via (at 138.571312 98.787) (size 0.8) (drill 0.4) (layers "F.Cu" "B.Cu") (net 2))
 (via (at 143.94489 98.787) (size 0.8) (drill 0.4) (layers "F.Cu" "B.Cu") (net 2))
 (via (at 213.801404 98.787) (size 0.8) (drill 0.4) (layers "F.Cu" "B.Cu") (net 2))
 (via (at 170.81278 98.787) (size 0.8) (drill 0.4) (layers "F.Cu" "B.Cu") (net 2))
 (via (at 197.68067 98.787) (size 0.8) (drill 0.4) (layers "F.Cu" "B.Cu") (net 2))
 (via (at 208.427826 98.787) (size 0.8) (drill 0.4) (layers "F.Cu" "B.Cu") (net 2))
 (segment (start 218.488 98.787) (end 115.123 98.787) (width 0.4) (layer "B.Cu") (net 2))
 (segment (start 220.035123 97.239877) (end 218.703 98.572) (width 0.4) (layer "B.Cu") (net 2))
 (segment (start 115.123 98.787) (end 114.729 99.181) (width 0.4) (layer "B.Cu") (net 2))
 (segment (start 165.439202 98.787) (end 164.974 98.787) (width 0.4) (layer "B.Cu") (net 2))
 (segment (start 218.703 98.572) (end 218.488 98.787) (width 0.4) (layer "B.Cu") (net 2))
 (segment (start 220.267867 97.239877) (end 220.035123 97.239877) (width 0.4) (layer "B.Cu") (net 2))
 (segment (start 164.974 98.787) (end 164.584 99.177) (width 0.4) (layer "B.Cu") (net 2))
 (segment (start 164.584 99.177) (end 163.911 99.177) (width 0.4) (layer "B.Cu") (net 2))
 (segment (start 114.729 99.181) (end 111.764 99.181) (width 0.4) (layer "B.Cu") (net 2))
 (segment (start 112.626 97.501) (end 113.707 97.501) (width 0.5) (layer "F.Cu") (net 3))
 (segment (start 141.83 97.439) (end 141.60389 97.66511) (width 0.5) (layer "F.Cu") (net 3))
 (segment (start 152.351046 97.458046) (end 152.351046 98.53) (width 0.5) (layer "F.Cu") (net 3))
 (segment (start 189.966092 97.489092) (end 189.966092 98.53) (width 0.5) (layer "F.Cu") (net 3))
 (segment (start 200.713248 97.755) (end 200.713248 98.53) (width 0.5) (layer "F.Cu") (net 3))
 (segment (start 146.977468 97.663468) (end 146.977468 98.53) (width 0.5) (layer "F.Cu") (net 3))
 (segment (start 206.402826 97.439) (end 206.086826 97.755) (width 0.5) (layer "F.Cu") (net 3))
 (segment (start 201.029248 97.439) (end 200.713248 97.755) (width 0.5) (layer "F.Cu") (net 3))
 (segment (start 216.528 97.439) (end 216.834 97.745) (width 0.5) (layer "F.Cu") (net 3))
 (segment (start 211.776404 97.439) (end 211.460404 97.755) (width 0.5) (layer "F.Cu") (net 3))
 (segment (start 216.528 97.439) (end 218.969 97.439) (width 0.5) (layer "F.Cu") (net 3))
 (segment (start 219.693 98.163) (end 219.693 98.53) (width 0.5) (layer "F.Cu") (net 3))
 (segment (start 216.834 97.745) (end 216.834 98.53) (width 0.5) (layer "F.Cu") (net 3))
 (segment (start 195.669 97.439) (end 195.33967 97.76833) (width 0.5) (layer "F.Cu") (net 3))
 (segment (start 164.994 97.439) (end 216.528 97.439) (width 0.5) (layer "F.Cu") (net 3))
 (segment (start 136.230312 97.873202) (end 136.230312 98.53) (width 0.5) (layer "F.Cu") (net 3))
 (segment (start 206.086826 97.755) (end 206.086826 98.53) (width 0.5) (layer "F.Cu") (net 3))
 (segment (start 114.736 97.755) (end 114.736 98.53) (width 0.5) (layer "F.Cu") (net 3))
 (segment (start 125.483156 97.873202) (end 125.483156 98.53) (width 0.5) (layer "F.Cu") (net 3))
 (segment (start 218.969 97.439) (end 219.693 98.163) (width 0.5) (layer "F.Cu") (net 3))
 (segment (start 173.845358 97.476358) (end 173.845358 98.53) (width 0.5) (layer "F.Cu") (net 3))
 (segment (start 135.79611 97.439) (end 136.230312 97.873202) (width 0.5) (layer "F.Cu") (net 3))
 (segment (start 125.048954 97.439) (end 125.483156 97.873202) (width 0.5) (layer "F.Cu") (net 3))
 (segment (start 157.724624 97.444624) (end 157.724624 98.53) (width 0.5) (layer "F.Cu") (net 3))
 (segment (start 179.218936 97.463064) (end 179.218936 98.53) (width 0.5) (layer "F.Cu") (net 3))
 (segment (start 130.422532 97.439) (end 130.856734 97.873202) (width 0.5) (layer "F.Cu") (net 3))
 (segment (start 163.098202 97.446798) (end 163.098202 98.53) (width 0.5) (layer "F.Cu") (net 3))
 (segment (start 184.592514 97.450514) (end 184.592514 98.53) (width 0.5) (layer "F.Cu") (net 3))
 (segment (start 195.33967 97.76833) (end 195.33967 98.53) (width 0.5) (layer "F.Cu") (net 3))
 (segment (start 115.052 97.439) (end 114.736 97.755) (width 0.5) (layer "F.Cu") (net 3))
 (segment (start 115.397 97.439) (end 112.688 97.439) (width 0.5) (layer "F.Cu") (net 3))
 (segment (start 115.397 97.439) (end 164.994 97.439) (width 0.5) (layer "F.Cu") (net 3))
 (segment (start 141.60389 97.66511) (end 141.60389 98.53) (width 0.5) (layer "F.Cu") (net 3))
 (segment (start 130.856734 97.873202) (end 130.856734 98.53) (width 0.5) (layer "F.Cu") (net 3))
 (segment (start 119.675376 97.439) (end 120.109578 97.873202) (width 0.5) (layer "F.Cu") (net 3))
 (segment (start 120.109578 97.873202) (end 120.109578 98.53) (width 0.5) (layer "F.Cu") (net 3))
 (segment (start 112.688 97.439) (end 112.626 97.501) (width 0.5) (layer "F.Cu") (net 3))
 (segment (start 168.47178 97.67622) (end 168.47178 98.53) (width 0.5) (layer "F.Cu") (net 3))
 (segment (start 211.460404 97.755) (end 211.460404 98.53) (width 0.5) (layer "F.Cu") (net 3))
 (via (at 113.505 97.479) (size 0.5) (drill 0.3) (layers "F.Cu" "B.Cu") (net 3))
 (via (at 111.744 97.479) (size 0.5) (drill 0.3) (layers "F.Cu" "B.Cu") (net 3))
 (via (at 112.6245 97.479) (size 0.5) (drill 0.3) (layers "F.Cu" "B.Cu") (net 3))
 (via (at 164.994 97.439) (size 0.8) (drill 0.4) (layers "F.Cu" "B.Cu") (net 3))
 (segment (start 166.648 97.821) (end 166.003 97.821) (width 0.5) (layer "B.Cu") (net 3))
 (segment (start 165.621 97.439) (end 164.994 97.439) (width 0.5) (layer "B.Cu") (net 3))
 (segment (start 166.003 97.821) (end 165.621 97.439) (width 0.5) (layer "B.Cu") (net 3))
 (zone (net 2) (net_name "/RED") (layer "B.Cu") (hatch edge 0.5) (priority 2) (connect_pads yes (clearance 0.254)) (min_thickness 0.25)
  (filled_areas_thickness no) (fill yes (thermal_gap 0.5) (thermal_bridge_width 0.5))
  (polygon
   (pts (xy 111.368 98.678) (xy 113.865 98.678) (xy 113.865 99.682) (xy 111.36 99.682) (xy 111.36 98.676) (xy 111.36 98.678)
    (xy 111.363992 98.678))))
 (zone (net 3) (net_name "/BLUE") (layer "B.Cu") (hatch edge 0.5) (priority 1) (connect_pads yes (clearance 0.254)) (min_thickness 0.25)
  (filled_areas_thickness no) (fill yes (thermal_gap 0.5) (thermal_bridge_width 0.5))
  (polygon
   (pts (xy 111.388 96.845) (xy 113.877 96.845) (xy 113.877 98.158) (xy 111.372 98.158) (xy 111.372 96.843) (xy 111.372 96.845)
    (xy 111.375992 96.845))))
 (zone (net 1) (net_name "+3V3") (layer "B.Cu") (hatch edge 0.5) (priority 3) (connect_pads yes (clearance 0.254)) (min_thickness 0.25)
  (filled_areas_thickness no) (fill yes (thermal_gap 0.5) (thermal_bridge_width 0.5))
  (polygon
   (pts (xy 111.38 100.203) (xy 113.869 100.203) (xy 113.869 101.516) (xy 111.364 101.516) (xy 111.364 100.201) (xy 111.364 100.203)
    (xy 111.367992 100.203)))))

